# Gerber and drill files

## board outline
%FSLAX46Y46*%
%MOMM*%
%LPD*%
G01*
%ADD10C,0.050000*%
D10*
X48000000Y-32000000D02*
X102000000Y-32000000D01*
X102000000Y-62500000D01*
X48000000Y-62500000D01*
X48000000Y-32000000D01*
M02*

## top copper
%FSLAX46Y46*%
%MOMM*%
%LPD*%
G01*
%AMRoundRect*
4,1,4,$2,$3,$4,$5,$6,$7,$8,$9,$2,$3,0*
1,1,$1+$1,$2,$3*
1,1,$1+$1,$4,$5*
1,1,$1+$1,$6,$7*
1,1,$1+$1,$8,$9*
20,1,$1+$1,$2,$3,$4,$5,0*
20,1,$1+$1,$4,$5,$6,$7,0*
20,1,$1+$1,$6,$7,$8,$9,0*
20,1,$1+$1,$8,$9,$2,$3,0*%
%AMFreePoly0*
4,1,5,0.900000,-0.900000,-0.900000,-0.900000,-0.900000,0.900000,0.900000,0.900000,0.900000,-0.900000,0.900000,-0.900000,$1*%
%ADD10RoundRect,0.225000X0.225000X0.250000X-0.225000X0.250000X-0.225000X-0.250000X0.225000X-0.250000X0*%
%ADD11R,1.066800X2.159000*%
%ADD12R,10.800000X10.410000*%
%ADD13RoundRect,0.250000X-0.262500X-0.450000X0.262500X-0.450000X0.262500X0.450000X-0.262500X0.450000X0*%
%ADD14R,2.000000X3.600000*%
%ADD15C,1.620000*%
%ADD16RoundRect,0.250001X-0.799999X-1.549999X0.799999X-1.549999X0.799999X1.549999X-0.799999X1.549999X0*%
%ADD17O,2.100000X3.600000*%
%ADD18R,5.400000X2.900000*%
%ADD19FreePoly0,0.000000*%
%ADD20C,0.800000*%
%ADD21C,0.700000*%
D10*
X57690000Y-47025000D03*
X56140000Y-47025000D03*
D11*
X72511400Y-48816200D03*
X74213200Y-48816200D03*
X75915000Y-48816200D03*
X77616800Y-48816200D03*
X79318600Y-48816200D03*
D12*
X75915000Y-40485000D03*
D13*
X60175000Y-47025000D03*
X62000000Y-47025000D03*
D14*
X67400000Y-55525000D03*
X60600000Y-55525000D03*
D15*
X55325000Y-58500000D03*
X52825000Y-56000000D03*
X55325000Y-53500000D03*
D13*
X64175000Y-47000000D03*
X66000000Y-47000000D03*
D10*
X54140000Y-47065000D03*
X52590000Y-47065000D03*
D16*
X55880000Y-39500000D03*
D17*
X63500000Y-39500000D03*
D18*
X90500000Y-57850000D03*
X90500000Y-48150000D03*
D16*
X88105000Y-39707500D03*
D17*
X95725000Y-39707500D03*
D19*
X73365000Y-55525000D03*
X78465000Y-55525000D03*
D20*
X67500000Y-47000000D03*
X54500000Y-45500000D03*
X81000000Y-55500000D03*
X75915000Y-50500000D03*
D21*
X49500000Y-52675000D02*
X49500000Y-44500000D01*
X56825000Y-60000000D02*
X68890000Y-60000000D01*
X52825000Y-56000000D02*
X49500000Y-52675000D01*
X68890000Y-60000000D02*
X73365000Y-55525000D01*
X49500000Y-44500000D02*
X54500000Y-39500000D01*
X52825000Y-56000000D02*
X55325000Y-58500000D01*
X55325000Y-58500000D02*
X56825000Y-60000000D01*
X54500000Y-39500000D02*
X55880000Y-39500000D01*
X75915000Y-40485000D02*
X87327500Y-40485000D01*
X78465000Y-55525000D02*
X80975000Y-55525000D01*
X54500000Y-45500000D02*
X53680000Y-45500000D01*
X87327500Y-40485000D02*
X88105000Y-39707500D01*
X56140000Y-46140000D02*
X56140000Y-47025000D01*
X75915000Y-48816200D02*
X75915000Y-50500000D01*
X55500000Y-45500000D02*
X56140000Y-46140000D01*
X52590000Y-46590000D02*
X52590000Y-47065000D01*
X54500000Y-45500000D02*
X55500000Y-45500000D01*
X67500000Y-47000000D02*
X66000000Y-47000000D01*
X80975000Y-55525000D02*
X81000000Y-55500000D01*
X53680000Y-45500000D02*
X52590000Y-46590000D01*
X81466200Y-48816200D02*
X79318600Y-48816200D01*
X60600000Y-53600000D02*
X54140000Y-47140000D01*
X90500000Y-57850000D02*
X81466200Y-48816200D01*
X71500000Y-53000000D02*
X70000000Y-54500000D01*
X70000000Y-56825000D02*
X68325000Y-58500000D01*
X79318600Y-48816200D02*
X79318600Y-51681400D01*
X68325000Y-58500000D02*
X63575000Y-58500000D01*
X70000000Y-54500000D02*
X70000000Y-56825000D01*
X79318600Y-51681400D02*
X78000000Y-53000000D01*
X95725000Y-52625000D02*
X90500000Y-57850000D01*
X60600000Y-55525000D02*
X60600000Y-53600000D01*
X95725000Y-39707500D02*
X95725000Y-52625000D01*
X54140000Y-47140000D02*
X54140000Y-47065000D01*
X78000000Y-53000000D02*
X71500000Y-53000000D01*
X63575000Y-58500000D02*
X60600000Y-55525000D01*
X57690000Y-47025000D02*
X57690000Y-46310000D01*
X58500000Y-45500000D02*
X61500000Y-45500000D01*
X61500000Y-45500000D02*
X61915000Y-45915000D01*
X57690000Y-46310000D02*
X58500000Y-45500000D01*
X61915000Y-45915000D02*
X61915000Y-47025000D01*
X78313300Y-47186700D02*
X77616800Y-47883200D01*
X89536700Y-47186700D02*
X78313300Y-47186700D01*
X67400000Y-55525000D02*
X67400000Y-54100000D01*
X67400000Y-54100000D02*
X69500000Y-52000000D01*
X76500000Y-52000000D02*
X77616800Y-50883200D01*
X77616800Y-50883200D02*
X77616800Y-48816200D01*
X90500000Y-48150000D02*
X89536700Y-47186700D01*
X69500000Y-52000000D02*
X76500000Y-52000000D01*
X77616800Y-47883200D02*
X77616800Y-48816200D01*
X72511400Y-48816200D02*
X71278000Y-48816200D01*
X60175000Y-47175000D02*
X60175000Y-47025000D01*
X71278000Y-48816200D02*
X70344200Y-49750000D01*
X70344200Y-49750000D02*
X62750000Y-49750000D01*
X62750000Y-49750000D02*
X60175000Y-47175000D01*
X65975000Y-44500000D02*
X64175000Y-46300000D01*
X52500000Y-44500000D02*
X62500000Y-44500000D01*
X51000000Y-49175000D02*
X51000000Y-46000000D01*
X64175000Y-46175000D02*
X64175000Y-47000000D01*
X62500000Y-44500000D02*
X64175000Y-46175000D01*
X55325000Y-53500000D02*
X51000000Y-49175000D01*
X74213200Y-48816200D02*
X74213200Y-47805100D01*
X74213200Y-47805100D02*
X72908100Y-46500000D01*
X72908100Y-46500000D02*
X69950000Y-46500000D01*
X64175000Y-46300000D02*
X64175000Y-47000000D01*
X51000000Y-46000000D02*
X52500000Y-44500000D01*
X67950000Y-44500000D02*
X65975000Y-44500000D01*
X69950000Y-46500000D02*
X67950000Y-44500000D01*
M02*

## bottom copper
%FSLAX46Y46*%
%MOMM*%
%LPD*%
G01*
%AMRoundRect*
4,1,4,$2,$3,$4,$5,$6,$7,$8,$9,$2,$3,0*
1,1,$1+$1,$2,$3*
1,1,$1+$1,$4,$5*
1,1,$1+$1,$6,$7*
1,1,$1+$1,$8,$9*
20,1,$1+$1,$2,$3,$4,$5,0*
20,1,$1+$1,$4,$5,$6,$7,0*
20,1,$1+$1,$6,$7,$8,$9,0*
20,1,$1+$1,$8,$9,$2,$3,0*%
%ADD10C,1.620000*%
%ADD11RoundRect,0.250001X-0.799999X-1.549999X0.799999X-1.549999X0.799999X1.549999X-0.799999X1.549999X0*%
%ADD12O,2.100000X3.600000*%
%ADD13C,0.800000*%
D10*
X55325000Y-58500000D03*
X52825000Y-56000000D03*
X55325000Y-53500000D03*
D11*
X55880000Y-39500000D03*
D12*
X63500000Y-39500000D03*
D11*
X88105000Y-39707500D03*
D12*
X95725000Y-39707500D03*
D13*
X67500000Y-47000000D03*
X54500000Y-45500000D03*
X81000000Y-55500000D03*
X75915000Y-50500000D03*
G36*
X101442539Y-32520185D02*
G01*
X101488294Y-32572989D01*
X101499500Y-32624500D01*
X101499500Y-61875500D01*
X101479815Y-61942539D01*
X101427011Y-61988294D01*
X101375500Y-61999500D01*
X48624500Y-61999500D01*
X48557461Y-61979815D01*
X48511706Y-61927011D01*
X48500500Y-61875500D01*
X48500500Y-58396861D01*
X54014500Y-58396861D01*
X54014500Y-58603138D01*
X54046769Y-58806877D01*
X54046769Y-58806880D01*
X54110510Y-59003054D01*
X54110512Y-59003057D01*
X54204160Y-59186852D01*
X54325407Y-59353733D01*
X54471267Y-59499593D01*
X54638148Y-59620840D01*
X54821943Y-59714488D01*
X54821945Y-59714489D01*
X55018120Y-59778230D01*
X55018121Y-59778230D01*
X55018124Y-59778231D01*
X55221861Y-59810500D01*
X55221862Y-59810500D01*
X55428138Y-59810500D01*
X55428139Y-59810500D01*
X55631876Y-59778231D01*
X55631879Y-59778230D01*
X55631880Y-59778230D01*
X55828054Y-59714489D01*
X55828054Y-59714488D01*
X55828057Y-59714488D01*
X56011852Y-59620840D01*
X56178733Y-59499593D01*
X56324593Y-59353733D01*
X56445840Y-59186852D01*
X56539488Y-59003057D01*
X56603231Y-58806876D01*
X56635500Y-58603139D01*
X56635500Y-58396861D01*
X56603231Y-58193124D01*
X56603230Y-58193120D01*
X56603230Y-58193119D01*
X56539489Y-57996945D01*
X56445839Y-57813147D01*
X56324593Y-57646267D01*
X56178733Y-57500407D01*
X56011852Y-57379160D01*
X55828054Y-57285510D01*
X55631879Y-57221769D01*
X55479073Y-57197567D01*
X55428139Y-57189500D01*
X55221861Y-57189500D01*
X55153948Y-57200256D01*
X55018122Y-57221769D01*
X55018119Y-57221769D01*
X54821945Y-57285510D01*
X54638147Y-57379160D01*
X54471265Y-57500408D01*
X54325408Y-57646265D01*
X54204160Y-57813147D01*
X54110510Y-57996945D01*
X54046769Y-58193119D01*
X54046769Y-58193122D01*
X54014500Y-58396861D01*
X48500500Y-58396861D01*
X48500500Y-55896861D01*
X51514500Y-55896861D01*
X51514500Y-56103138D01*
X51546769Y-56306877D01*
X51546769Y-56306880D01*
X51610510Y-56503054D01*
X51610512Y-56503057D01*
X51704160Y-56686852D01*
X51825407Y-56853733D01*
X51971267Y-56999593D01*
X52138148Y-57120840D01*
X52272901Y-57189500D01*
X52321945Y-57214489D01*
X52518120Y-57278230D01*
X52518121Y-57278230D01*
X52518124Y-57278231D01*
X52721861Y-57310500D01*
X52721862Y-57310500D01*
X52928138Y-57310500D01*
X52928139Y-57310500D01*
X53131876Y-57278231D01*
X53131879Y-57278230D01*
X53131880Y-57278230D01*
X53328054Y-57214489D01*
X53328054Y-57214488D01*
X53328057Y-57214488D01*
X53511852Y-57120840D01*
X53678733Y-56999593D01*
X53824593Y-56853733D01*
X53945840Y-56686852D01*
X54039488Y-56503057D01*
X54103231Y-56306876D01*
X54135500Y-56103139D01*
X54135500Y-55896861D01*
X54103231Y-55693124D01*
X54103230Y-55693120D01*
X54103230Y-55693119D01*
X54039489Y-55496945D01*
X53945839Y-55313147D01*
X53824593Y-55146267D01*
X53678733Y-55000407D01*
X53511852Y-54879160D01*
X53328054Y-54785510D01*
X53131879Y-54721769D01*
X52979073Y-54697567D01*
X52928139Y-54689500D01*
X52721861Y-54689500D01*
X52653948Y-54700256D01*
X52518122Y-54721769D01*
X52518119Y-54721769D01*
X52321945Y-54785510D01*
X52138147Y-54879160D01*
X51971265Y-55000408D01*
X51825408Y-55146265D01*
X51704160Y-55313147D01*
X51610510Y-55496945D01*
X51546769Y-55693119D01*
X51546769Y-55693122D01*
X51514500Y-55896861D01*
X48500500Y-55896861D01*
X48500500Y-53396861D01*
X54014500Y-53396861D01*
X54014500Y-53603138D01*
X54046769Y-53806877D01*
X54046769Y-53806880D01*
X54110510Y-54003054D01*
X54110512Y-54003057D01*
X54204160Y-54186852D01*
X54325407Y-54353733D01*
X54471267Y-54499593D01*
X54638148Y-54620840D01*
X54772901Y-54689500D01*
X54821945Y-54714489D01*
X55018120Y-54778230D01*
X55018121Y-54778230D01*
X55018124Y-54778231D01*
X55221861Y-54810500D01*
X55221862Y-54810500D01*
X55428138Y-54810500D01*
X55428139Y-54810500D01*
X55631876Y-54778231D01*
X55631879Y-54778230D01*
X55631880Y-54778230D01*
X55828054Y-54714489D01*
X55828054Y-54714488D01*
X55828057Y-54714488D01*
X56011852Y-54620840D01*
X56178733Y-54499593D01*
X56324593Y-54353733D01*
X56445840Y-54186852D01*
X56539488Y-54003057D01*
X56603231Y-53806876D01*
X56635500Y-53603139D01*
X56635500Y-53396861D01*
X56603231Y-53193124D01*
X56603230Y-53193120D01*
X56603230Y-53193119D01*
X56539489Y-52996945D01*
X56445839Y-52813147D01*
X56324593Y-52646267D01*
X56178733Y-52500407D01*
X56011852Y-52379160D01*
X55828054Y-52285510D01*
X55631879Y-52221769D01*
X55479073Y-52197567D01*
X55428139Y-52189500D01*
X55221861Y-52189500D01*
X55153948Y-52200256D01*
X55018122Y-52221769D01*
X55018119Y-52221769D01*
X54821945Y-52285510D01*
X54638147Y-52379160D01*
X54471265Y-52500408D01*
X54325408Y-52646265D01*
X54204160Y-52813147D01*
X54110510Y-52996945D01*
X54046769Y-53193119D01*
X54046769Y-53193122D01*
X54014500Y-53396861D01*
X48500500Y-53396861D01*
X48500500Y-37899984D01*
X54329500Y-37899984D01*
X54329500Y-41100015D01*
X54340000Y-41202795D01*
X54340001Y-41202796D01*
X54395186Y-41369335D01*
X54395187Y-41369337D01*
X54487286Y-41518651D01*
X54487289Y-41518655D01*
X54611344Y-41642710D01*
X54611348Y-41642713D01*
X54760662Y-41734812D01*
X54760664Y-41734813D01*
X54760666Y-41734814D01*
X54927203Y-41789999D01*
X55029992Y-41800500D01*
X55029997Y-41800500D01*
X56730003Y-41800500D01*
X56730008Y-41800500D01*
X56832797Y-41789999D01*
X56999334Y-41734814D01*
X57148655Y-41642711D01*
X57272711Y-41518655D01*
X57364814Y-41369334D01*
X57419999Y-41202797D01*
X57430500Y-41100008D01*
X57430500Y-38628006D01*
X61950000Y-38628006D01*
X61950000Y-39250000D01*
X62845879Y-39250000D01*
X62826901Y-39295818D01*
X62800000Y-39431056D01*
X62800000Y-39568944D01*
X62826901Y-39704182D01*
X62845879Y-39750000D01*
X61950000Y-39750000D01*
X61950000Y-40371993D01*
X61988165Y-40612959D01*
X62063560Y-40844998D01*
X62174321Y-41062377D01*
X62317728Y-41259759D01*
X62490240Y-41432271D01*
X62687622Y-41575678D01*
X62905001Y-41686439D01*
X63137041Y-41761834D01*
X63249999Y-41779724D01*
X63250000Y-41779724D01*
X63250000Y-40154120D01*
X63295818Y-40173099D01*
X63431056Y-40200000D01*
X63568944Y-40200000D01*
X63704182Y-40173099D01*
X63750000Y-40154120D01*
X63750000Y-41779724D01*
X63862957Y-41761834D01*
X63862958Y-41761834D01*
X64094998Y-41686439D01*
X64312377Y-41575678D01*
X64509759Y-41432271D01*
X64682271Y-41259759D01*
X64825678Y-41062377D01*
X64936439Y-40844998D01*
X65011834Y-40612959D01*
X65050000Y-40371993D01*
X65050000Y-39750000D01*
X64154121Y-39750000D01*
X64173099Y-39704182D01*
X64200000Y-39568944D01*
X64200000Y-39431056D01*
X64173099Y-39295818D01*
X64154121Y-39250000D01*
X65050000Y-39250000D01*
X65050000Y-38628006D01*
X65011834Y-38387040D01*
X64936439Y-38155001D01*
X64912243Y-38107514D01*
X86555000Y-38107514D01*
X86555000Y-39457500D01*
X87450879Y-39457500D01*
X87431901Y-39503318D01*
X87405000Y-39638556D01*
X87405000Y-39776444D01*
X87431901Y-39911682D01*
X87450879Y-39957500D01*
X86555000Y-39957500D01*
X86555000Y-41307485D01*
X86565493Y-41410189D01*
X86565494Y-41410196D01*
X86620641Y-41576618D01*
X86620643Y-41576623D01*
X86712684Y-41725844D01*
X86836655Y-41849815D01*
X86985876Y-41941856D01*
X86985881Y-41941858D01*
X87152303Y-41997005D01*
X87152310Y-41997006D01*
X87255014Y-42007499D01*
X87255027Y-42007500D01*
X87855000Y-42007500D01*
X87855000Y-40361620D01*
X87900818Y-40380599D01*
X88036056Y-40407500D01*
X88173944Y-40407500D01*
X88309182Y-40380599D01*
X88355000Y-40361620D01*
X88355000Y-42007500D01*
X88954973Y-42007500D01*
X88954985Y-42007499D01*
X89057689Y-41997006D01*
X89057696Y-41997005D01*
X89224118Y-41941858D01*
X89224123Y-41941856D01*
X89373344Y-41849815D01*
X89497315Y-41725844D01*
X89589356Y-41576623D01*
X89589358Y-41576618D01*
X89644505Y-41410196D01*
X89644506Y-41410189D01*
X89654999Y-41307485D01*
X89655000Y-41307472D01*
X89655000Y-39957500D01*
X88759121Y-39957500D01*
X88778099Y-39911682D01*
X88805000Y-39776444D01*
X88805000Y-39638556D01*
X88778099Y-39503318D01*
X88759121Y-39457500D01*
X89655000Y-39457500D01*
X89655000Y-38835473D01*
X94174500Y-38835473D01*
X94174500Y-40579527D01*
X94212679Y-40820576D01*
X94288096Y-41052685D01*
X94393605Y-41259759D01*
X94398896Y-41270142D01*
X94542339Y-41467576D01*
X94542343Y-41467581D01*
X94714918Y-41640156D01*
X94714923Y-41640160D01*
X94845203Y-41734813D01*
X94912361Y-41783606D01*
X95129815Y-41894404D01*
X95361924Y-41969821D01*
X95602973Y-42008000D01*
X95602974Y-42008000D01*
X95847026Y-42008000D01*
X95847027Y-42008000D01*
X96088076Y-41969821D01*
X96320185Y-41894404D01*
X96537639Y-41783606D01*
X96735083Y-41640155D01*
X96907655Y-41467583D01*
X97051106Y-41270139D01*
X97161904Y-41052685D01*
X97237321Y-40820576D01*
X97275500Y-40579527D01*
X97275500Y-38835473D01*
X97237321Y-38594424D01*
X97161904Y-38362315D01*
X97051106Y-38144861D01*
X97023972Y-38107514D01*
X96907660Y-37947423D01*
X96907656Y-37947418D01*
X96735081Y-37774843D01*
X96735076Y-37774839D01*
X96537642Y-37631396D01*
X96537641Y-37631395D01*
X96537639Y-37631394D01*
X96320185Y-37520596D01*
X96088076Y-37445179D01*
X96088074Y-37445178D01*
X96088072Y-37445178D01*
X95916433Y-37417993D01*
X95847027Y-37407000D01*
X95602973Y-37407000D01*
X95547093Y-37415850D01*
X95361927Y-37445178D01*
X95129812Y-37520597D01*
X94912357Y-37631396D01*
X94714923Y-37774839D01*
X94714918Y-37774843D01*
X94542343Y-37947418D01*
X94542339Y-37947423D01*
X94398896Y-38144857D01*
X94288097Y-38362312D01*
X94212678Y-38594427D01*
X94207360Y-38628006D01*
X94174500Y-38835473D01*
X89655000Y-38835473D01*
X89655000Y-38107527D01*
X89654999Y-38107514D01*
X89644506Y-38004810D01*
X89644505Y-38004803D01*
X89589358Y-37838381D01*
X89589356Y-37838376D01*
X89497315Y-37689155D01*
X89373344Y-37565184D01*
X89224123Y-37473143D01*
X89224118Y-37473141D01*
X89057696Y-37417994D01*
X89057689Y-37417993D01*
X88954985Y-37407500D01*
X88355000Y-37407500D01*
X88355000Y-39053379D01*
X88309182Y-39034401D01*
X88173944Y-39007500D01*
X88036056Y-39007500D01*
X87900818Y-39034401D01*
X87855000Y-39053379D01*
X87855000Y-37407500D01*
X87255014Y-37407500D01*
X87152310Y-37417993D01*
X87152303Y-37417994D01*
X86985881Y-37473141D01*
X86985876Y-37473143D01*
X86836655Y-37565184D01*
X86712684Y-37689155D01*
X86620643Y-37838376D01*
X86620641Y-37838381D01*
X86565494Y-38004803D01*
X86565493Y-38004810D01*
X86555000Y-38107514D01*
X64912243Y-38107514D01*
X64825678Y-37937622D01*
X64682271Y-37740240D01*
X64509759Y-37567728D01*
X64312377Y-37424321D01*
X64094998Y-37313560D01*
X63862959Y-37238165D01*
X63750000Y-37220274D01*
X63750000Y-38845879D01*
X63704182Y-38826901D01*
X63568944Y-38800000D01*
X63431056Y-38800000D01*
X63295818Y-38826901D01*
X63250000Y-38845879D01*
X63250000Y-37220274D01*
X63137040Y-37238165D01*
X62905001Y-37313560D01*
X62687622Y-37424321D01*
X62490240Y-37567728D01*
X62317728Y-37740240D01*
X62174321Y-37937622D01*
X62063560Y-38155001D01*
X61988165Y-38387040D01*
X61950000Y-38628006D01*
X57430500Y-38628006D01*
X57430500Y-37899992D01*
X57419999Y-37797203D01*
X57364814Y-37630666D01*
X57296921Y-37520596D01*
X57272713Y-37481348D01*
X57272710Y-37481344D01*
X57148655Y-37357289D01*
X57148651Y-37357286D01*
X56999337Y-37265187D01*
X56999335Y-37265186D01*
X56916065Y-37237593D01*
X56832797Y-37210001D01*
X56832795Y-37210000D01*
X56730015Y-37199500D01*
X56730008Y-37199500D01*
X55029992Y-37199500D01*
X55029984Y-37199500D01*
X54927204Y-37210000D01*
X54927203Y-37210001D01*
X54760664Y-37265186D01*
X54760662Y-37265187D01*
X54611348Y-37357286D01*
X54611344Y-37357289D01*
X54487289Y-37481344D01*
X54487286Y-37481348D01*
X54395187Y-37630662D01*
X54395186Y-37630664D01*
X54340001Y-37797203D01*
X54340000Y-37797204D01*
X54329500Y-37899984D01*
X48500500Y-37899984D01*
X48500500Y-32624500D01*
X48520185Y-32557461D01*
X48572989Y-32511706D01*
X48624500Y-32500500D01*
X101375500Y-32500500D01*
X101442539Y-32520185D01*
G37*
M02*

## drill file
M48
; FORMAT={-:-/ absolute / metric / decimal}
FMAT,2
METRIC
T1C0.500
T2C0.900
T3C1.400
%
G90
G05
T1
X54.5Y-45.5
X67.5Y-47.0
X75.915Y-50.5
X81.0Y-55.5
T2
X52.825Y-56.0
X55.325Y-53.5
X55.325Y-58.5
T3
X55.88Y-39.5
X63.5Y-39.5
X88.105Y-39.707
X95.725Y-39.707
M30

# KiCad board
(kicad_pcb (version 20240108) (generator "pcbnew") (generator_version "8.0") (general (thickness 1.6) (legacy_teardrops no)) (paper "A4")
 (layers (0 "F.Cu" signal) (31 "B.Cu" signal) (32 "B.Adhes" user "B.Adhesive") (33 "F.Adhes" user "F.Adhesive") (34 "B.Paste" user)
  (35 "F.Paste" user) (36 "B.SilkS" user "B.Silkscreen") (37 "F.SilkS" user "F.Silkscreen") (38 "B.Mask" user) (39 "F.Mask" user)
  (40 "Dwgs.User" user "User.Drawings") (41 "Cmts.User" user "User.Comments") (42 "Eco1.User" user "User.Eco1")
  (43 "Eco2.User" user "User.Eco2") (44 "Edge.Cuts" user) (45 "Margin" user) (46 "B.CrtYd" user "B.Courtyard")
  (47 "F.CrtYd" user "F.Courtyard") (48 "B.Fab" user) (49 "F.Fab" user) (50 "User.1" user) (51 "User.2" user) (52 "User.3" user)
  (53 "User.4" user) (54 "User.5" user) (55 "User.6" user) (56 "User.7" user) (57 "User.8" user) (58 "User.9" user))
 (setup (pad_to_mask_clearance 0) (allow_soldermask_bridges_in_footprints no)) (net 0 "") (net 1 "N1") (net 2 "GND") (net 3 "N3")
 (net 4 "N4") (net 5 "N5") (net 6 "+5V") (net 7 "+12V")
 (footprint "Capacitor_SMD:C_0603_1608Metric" (layer "F.Cu") (at 56.915 47.025 180)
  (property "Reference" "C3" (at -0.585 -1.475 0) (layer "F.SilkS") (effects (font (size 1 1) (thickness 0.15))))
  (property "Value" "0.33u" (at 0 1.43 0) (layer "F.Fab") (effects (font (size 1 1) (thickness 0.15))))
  (pad "1" smd roundrect (at -0.775 0 180) (size 0.9 0.95) (layers "F.Cu" "F.Paste" "F.Mask") (roundrect_rratio 0.25) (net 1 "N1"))
  (pad "2" smd roundrect (at 0.775 0 180) (size 0.9 0.95) (layers "F.Cu" "F.Paste" "F.Mask") (roundrect_rratio 0.25) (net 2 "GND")))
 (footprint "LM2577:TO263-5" (layer "F.Cu") (at 75.915 43.025)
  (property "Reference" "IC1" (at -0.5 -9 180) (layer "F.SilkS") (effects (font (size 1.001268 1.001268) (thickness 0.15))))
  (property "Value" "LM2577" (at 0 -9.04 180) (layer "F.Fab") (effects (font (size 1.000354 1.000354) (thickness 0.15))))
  (pad "1" smd rect (at -3.4036 5.7912) (size 1.0668 2.159) (layers "F.Cu" "F.Paste" "F.Mask") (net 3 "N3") (solder_mask_margin 0.102))
  (pad "2" smd rect (at -1.7018 5.7912) (size 1.0668 2.159) (layers "F.Cu" "F.Paste" "F.Mask") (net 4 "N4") (solder_mask_margin 0.102))
  (pad "3" smd rect (at 0 5.7912) (size 1.0668 2.159) (layers "F.Cu" "F.Paste" "F.Mask") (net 2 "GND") (solder_mask_margin 0.102))
  (pad "4" smd rect (at 1.7018 5.7912) (size 1.0668 2.159) (layers "F.Cu" "F.Paste" "F.Mask") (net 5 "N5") (solder_mask_margin 0.102))
  (pad "5" smd rect (at 3.4036 5.7912) (size 1.0668 2.159) (layers "F.Cu" "F.Paste" "F.Mask") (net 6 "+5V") (solder_mask_margin 0.102))
  (pad "6" smd rect (at 0 -2.54) (size 10.8 10.41) (layers "F.Cu" "F.Paste" "F.Mask") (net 2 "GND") (solder_mask_margin 0.102)))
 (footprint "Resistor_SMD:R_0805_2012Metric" (layer "F.Cu") (at 61.0875 47.025)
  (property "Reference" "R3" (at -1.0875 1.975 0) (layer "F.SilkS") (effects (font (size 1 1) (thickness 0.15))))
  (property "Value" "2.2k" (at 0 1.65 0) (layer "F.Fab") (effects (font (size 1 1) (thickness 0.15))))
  (pad "1" smd roundrect (at -0.9125 0) (size 1.025 1.4) (layers "F.Cu" "F.Paste" "F.Mask") (roundrect_rratio 0.243902) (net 3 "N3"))
  (pad "2" smd roundrect (at 0.9125 0) (size 1.025 1.4) (layers "F.Cu" "F.Paste" "F.Mask") (roundrect_rratio 0.243902) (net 1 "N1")))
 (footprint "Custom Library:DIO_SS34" (layer "F.Cu") (at 64 55.525)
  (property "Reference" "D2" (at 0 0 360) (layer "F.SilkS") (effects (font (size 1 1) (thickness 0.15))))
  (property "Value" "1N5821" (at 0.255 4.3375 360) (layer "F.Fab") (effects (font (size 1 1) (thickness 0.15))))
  (pad "A" smd rect (at 3.4 0) (size 2 3.6) (layers "F.Cu" "F.Paste" "F.Mask") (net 5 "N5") (solder_mask_margin 0.102))
  (pad "C" smd rect (at -3.4 0) (size 2 3.6) (layers "F.Cu" "F.Paste" "F.Mask") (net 6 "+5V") (solder_mask_margin 0.102)))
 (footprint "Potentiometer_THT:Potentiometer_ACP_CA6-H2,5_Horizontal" (layer "F.Cu") (at 55.325 58.5 180)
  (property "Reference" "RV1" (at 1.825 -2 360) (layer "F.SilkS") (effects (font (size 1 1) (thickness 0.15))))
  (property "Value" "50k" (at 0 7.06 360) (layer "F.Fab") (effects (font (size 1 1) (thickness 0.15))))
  (pad "1" thru_hole circle (at 0 0 180) (size 1.62 1.62) (drill 0.9) (layers "*.Cu" "*.Mask") (remove_unused_layers no) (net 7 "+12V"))
  (pad "2" thru_hole circle (at 2.5 2.5 180) (size 1.62 1.62) (drill 0.9) (layers "*.Cu" "*.Mask") (remove_unused_layers no) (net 7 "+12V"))
  (pad "3" thru_hole circle (at 0 5 180) (size 1.62 1.62) (drill 0.9) (layers "*.Cu" "*.Mask") (remove_unused_layers no) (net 4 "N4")))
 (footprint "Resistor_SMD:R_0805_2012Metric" (layer "F.Cu") (at 65.0875 47)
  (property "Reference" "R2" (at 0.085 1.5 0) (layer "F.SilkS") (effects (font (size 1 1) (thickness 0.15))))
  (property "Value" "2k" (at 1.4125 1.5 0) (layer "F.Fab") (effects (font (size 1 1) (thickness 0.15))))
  (pad "1" smd roundrect (at -0.9125 0) (size 1.025 1.4) (layers "F.Cu" "F.Paste" "F.Mask") (roundrect_rratio 0.243902) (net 4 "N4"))
  (pad "2" smd roundrect (at 0.9125 0) (size 1.025 1.4) (layers "F.Cu" "F.Paste" "F.Mask") (roundrect_rratio 0.243902) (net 2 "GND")))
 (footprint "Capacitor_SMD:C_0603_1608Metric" (layer "F.Cu") (at 53.365 47.065 180)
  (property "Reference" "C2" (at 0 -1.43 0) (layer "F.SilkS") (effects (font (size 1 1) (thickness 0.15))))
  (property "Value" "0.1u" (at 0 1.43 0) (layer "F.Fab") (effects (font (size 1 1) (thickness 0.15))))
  (pad "1" smd roundrect (at -0.775 0 180) (size 0.9 0.95) (layers "F.Cu" "F.Paste" "F.Mask") (roundrect_rratio 0.25) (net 6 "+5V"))
  (pad "2" smd roundrect (at 0.775 0 180) (size 0.9 0.95) (layers "F.Cu" "F.Paste" "F.Mask") (roundrect_rratio 0.25) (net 2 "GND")))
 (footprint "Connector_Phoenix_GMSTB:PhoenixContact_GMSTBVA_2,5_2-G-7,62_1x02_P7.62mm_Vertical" (layer "F.Cu") (at 55.88 39.5)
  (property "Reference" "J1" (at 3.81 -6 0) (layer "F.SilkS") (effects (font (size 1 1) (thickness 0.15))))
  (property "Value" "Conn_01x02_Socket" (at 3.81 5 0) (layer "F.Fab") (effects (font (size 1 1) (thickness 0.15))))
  (pad "1" thru_hole roundrect (at 0 0) (size 2.1 3.6) (drill 1.4) (layers "*.Cu" "*.Mask") (remove_unused_layers no)
   (roundrect_rratio 0.119048) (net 7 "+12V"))
  (pad "2" thru_hole oval (at 7.62 0) (size 2.1 3.6) (drill 1.4) (layers "*.Cu" "*.Mask") (remove_unused_layers no) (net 2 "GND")))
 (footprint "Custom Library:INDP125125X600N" (layer "F.Cu") (at 90.5 53 90)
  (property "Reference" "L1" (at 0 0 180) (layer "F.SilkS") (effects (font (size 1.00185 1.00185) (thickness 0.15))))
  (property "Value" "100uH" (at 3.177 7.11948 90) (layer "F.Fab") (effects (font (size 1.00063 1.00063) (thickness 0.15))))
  (pad "1" smd rect (at -4.85 0 90) (size 2.9 5.4) (layers "F.Cu" "F.Paste" "F.Mask") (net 6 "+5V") (solder_mask_margin 0.102))
  (pad "2" smd rect (at 4.85 0 90) (size 2.9 5.4) (layers "F.Cu" "F.Paste" "F.Mask") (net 5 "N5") (solder_mask_margin 0.102)))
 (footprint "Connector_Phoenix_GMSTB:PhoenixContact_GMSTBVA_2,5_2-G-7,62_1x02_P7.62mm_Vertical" (layer "F.Cu") (at 88.105 39.7075)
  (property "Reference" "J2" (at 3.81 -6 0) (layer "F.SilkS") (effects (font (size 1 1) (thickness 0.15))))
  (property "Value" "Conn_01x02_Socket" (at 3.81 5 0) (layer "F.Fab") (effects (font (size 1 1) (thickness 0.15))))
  (pad "1" thru_hole roundrect (at 0 0) (size 2.1 3.6) (drill 1.4) (layers "*.Cu" "*.Mask") (remove_unused_layers no)
   (roundrect_rratio 0.119048) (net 2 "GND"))
  (pad "2" thru_hole oval (at 7.62 0) (size 2.1 3.6) (drill 1.4) (layers "*.Cu" "*.Mask") (remove_unused_layers no) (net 6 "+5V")))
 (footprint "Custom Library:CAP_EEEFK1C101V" (layer "F.Cu") (at 75.915 55.525)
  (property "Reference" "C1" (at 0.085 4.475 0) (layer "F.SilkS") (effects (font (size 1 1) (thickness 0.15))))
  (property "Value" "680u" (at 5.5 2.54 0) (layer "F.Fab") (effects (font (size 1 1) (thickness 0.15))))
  (pad "1" smd custom (at -2.55 0) (size 1.8 1.8) (layers "F.Cu") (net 7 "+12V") (options (clearance outline) (anchor rect)) (primitives))
  (pad "2" smd custom (at 2.55 0) (size 1.8 1.8) (layers "F.Cu") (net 2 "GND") (options (clearance outline) (anchor rect)) (primitives)))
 (gr_rect (start 48 32) (end 102 62.5) (stroke (width 0.05) (type default)) (fill none) (layer "Edge.Cuts"))
 (segment (start 49.5 52.675) (end 49.5 44.5) (width 0.7) (layer "F.Cu") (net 7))
 (segment (start 56.825 60) (end 68.89 60) (width 0.7) (layer "F.Cu") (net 7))
 (segment (start 52.825 56) (end 49.5 52.675) (width 0.7) (layer "F.Cu") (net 7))
 (segment (start 68.89 60) (end 73.365 55.525) (width 0.7) (layer "F.Cu") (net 7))
 (segment (start 49.5 44.5) (end 54.5 39.5) (width 0.7) (layer "F.Cu") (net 7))
 (segment (start 52.825 56) (end 55.325 58.5) (width 0.7) (layer "F.Cu") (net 7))
 (segment (start 55.325 58.5) (end 56.825 60) (width 0.7) (layer "F.Cu") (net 7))
 (segment (start 54.5 39.5) (end 55.88 39.5) (width 0.7) (layer "F.Cu") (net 7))
 (segment (start 75.915 40.485) (end 87.3275 40.485) (width 0.7) (layer "F.Cu") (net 2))
 (segment (start 78.465 55.525) (end 80.975 55.525) (width 0.7) (layer "F.Cu") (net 2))
 (segment (start 54.5 45.5) (end 53.68 45.5) (width 0.7) (layer "F.Cu") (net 2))
 (segment (start 87.3275 40.485) (end 88.105 39.7075) (width 0.7) (layer "F.Cu") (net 2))
 (segment (start 56.14 46.14) (end 56.14 47.025) (width 0.7) (layer "F.Cu") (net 2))
 (segment (start 75.915 48.8162) (end 75.915 50.5) (width 0.7) (layer "F.Cu") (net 2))
 (segment (start 55.5 45.5) (end 56.14 46.14) (width 0.7) (layer "F.Cu") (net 2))
 (segment (start 52.59 46.59) (end 52.59 47.065) (width 0.7) (layer "F.Cu") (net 2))
 (segment (start 54.5 45.5) (end 55.5 45.5) (width 0.7) (layer "F.Cu") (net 2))
 (segment (start 67.5 47) (end 66 47) (width 0.7) (layer "F.Cu") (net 2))
 (segment (start 80.975 55.525) (end 81 55.5) (width 0.7) (layer "F.Cu") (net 2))
 (segment (start 53.68 45.5) (end 52.59 46.59) (width 0.7) (layer "F.Cu") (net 2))
 (via (at 67.5 47) (size 0.8) (drill 0.5) (layers "F.Cu" "B.Cu") (free yes) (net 2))
 (via (at 54.5 45.5) (size 0.8) (drill 0.5) (layers "F.Cu" "B.Cu") (free yes) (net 2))
 (via (at 81 55.5) (size 0.8) (drill 0.5) (layers "F.Cu" "B.Cu") (free yes) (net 2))
 (via (at 75.915 50.5) (size 0.8) (drill 0.5) (layers "F.Cu" "B.Cu") (free yes) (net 2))
 (segment (start 81.4662 48.8162) (end 79.3186 48.8162) (width 0.7) (layer "F.Cu") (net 6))
 (segment (start 60.6 53.6) (end 54.14 47.14) (width 0.7) (layer "F.Cu") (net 6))
 (segment (start 90.5 57.85) (end 81.4662 48.8162) (width 0.7) (layer "F.Cu") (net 6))
 (segment (start 71.5 53) (end 70 54.5) (width 0.7) (layer "F.Cu") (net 6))
 (segment (start 70 56.825) (end 68.325 58.5) (width 0.7) (layer "F.Cu") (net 6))
 (segment (start 79.3186 48.8162) (end 79.3186 51.6814) (width 0.7) (layer "F.Cu") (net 6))
 (segment (start 68.325 58.5) (end 63.575 58.5) (width 0.7) (layer "F.Cu") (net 6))
 (segment (start 70 54.5) (end 70 56.825) (width 0.7) (layer "F.Cu") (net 6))
 (segment (start 79.3186 51.6814) (end 78 53) (width 0.7) (layer "F.Cu") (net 6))
 (segment (start 95.725 52.625) (end 90.5 57.85) (width 0.7) (layer "F.Cu") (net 6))
 (segment (start 60.6 55.525) (end 60.6 53.6) (width 0.7) (layer "F.Cu") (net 6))
 (segment (start 95.725 39.7075) (end 95.725 52.625) (width 0.7) (layer "F.Cu") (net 6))
 (segment (start 54.14 47.14) (end 54.14 47.065) (width 0.7) (layer "F.Cu") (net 6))
 (segment (start 78 53) (end 71.5 53) (width 0.7) (layer "F.Cu") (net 6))
 (segment (start 63.575 58.5) (end 60.6 55.525) (width 0.7) (layer "F.Cu") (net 6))
 (segment (start 57.69 47.025) (end 57.69 46.31) (width 0.7) (layer "F.Cu") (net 1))
 (segment (start 58.5 45.5) (end 61.5 45.5) (width 0.7) (layer "F.Cu") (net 1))
 (segment (start 61.5 45.5) (end 61.915 45.915) (width 0.7) (layer "F.Cu") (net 1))
 (segment (start 57.69 46.31) (end 58.5 45.5) (width 0.7) (layer "F.Cu") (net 1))
 (segment (start 61.915 45.915) (end 61.915 47.025) (width 0.7) (layer "F.Cu") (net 1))
 (segment (start 78.3133 47.1867) (end 77.6168 47.8832) (width 0.7) (layer "F.Cu") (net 5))
 (segment (start 89.5367 47.1867) (end 78.3133 47.1867) (width 0.7) (layer "F.Cu") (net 5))
 (segment (start 67.4 55.525) (end 67.4 54.1) (width 0.7) (layer "F.Cu") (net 5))
 (segment (start 67.4 54.1) (end 69.5 52) (width 0.7) (layer "F.Cu") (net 5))
 (segment (start 76.5 52) (end 77.6168 50.8832) (width 0.7) (layer "F.Cu") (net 5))
 (segment (start 77.6168 50.8832) (end 77.6168 48.8162) (width 0.7) (layer "F.Cu") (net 5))
 (segment (start 90.5 48.15) (end 89.5367 47.1867) (width 0.7) (layer "F.Cu") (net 5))
 (segment (start 69.5 52) (end 76.5 52) (width 0.7) (layer "F.Cu") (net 5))
 (segment (start 77.6168 47.8832) (end 77.6168 48.8162) (width 0.7) (layer "F.Cu") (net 5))
 (segment (start 72.5114 48.8162) (end 71.278 48.8162) (width 0.7) (layer "F.Cu") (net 3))
 (segment (start 60.175 47.175) (end 60.175 47.025) (width 0.7) (layer "F.Cu") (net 3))
 (segment (start 71.278 48.8162) (end 70.3442 49.75) (width 0.7) (layer "F.Cu") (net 3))
 (segment (start 70.3442 49.75) (end 62.75 49.75) (width 0.7) (layer "F.Cu") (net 3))
 (segment (start 62.75 49.75) (end 60.175 47.175) (width 0.7) (layer "F.Cu") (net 3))
 (segment (start 65.975 44.5) (end 64.175 46.3) (width 0.7) (layer "F.Cu") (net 4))
 (segment (start 52.5 44.5) (end 62.5 44.5) (width 0.7) (layer "F.Cu") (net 4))
 (segment (start 51 49.175) (end 51 46) (width 0.7) (layer "F.Cu") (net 4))
 (segment (start 64.175 46.175) (end 64.175 47) (width 0.7) (layer "F.Cu") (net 4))
 (segment (start 62.5 44.5) (end 64.175 46.175) (width 0.7) (layer "F.Cu") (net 4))
 (segment (start 55.325 53.5) (end 51 49.175) (width 0.7) (layer "F.Cu") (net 4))
 (segment (start 74.2132 48.8162) (end 74.2132 47.8051) (width 0.7) (layer "F.Cu") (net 4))
 (segment (start 74.2132 47.8051) (end 72.9081 46.5) (width 0.7) (layer "F.Cu") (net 4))
 (segment (start 72.9081 46.5) (end 69.95 46.5) (width 0.7) (layer "F.Cu") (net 4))
 (segment (start 64.175 46.3) (end 64.175 47) (width 0.7) (layer "F.Cu") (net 4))
 (segment (start 51 46) (end 52.5 44.5) (width 0.7) (layer "F.Cu") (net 4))
 (segment (start 67.95 44.5) (end 65.975 44.5) (width 0.7) (layer "F.Cu") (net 4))
 (segment (start 69.95 46.5) (end 67.95 44.5) (width 0.7) (layer "F.Cu") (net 4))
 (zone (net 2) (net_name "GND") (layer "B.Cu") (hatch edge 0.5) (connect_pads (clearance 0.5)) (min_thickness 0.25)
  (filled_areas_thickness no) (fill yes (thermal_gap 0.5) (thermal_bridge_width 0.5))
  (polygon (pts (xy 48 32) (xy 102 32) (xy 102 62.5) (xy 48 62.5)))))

